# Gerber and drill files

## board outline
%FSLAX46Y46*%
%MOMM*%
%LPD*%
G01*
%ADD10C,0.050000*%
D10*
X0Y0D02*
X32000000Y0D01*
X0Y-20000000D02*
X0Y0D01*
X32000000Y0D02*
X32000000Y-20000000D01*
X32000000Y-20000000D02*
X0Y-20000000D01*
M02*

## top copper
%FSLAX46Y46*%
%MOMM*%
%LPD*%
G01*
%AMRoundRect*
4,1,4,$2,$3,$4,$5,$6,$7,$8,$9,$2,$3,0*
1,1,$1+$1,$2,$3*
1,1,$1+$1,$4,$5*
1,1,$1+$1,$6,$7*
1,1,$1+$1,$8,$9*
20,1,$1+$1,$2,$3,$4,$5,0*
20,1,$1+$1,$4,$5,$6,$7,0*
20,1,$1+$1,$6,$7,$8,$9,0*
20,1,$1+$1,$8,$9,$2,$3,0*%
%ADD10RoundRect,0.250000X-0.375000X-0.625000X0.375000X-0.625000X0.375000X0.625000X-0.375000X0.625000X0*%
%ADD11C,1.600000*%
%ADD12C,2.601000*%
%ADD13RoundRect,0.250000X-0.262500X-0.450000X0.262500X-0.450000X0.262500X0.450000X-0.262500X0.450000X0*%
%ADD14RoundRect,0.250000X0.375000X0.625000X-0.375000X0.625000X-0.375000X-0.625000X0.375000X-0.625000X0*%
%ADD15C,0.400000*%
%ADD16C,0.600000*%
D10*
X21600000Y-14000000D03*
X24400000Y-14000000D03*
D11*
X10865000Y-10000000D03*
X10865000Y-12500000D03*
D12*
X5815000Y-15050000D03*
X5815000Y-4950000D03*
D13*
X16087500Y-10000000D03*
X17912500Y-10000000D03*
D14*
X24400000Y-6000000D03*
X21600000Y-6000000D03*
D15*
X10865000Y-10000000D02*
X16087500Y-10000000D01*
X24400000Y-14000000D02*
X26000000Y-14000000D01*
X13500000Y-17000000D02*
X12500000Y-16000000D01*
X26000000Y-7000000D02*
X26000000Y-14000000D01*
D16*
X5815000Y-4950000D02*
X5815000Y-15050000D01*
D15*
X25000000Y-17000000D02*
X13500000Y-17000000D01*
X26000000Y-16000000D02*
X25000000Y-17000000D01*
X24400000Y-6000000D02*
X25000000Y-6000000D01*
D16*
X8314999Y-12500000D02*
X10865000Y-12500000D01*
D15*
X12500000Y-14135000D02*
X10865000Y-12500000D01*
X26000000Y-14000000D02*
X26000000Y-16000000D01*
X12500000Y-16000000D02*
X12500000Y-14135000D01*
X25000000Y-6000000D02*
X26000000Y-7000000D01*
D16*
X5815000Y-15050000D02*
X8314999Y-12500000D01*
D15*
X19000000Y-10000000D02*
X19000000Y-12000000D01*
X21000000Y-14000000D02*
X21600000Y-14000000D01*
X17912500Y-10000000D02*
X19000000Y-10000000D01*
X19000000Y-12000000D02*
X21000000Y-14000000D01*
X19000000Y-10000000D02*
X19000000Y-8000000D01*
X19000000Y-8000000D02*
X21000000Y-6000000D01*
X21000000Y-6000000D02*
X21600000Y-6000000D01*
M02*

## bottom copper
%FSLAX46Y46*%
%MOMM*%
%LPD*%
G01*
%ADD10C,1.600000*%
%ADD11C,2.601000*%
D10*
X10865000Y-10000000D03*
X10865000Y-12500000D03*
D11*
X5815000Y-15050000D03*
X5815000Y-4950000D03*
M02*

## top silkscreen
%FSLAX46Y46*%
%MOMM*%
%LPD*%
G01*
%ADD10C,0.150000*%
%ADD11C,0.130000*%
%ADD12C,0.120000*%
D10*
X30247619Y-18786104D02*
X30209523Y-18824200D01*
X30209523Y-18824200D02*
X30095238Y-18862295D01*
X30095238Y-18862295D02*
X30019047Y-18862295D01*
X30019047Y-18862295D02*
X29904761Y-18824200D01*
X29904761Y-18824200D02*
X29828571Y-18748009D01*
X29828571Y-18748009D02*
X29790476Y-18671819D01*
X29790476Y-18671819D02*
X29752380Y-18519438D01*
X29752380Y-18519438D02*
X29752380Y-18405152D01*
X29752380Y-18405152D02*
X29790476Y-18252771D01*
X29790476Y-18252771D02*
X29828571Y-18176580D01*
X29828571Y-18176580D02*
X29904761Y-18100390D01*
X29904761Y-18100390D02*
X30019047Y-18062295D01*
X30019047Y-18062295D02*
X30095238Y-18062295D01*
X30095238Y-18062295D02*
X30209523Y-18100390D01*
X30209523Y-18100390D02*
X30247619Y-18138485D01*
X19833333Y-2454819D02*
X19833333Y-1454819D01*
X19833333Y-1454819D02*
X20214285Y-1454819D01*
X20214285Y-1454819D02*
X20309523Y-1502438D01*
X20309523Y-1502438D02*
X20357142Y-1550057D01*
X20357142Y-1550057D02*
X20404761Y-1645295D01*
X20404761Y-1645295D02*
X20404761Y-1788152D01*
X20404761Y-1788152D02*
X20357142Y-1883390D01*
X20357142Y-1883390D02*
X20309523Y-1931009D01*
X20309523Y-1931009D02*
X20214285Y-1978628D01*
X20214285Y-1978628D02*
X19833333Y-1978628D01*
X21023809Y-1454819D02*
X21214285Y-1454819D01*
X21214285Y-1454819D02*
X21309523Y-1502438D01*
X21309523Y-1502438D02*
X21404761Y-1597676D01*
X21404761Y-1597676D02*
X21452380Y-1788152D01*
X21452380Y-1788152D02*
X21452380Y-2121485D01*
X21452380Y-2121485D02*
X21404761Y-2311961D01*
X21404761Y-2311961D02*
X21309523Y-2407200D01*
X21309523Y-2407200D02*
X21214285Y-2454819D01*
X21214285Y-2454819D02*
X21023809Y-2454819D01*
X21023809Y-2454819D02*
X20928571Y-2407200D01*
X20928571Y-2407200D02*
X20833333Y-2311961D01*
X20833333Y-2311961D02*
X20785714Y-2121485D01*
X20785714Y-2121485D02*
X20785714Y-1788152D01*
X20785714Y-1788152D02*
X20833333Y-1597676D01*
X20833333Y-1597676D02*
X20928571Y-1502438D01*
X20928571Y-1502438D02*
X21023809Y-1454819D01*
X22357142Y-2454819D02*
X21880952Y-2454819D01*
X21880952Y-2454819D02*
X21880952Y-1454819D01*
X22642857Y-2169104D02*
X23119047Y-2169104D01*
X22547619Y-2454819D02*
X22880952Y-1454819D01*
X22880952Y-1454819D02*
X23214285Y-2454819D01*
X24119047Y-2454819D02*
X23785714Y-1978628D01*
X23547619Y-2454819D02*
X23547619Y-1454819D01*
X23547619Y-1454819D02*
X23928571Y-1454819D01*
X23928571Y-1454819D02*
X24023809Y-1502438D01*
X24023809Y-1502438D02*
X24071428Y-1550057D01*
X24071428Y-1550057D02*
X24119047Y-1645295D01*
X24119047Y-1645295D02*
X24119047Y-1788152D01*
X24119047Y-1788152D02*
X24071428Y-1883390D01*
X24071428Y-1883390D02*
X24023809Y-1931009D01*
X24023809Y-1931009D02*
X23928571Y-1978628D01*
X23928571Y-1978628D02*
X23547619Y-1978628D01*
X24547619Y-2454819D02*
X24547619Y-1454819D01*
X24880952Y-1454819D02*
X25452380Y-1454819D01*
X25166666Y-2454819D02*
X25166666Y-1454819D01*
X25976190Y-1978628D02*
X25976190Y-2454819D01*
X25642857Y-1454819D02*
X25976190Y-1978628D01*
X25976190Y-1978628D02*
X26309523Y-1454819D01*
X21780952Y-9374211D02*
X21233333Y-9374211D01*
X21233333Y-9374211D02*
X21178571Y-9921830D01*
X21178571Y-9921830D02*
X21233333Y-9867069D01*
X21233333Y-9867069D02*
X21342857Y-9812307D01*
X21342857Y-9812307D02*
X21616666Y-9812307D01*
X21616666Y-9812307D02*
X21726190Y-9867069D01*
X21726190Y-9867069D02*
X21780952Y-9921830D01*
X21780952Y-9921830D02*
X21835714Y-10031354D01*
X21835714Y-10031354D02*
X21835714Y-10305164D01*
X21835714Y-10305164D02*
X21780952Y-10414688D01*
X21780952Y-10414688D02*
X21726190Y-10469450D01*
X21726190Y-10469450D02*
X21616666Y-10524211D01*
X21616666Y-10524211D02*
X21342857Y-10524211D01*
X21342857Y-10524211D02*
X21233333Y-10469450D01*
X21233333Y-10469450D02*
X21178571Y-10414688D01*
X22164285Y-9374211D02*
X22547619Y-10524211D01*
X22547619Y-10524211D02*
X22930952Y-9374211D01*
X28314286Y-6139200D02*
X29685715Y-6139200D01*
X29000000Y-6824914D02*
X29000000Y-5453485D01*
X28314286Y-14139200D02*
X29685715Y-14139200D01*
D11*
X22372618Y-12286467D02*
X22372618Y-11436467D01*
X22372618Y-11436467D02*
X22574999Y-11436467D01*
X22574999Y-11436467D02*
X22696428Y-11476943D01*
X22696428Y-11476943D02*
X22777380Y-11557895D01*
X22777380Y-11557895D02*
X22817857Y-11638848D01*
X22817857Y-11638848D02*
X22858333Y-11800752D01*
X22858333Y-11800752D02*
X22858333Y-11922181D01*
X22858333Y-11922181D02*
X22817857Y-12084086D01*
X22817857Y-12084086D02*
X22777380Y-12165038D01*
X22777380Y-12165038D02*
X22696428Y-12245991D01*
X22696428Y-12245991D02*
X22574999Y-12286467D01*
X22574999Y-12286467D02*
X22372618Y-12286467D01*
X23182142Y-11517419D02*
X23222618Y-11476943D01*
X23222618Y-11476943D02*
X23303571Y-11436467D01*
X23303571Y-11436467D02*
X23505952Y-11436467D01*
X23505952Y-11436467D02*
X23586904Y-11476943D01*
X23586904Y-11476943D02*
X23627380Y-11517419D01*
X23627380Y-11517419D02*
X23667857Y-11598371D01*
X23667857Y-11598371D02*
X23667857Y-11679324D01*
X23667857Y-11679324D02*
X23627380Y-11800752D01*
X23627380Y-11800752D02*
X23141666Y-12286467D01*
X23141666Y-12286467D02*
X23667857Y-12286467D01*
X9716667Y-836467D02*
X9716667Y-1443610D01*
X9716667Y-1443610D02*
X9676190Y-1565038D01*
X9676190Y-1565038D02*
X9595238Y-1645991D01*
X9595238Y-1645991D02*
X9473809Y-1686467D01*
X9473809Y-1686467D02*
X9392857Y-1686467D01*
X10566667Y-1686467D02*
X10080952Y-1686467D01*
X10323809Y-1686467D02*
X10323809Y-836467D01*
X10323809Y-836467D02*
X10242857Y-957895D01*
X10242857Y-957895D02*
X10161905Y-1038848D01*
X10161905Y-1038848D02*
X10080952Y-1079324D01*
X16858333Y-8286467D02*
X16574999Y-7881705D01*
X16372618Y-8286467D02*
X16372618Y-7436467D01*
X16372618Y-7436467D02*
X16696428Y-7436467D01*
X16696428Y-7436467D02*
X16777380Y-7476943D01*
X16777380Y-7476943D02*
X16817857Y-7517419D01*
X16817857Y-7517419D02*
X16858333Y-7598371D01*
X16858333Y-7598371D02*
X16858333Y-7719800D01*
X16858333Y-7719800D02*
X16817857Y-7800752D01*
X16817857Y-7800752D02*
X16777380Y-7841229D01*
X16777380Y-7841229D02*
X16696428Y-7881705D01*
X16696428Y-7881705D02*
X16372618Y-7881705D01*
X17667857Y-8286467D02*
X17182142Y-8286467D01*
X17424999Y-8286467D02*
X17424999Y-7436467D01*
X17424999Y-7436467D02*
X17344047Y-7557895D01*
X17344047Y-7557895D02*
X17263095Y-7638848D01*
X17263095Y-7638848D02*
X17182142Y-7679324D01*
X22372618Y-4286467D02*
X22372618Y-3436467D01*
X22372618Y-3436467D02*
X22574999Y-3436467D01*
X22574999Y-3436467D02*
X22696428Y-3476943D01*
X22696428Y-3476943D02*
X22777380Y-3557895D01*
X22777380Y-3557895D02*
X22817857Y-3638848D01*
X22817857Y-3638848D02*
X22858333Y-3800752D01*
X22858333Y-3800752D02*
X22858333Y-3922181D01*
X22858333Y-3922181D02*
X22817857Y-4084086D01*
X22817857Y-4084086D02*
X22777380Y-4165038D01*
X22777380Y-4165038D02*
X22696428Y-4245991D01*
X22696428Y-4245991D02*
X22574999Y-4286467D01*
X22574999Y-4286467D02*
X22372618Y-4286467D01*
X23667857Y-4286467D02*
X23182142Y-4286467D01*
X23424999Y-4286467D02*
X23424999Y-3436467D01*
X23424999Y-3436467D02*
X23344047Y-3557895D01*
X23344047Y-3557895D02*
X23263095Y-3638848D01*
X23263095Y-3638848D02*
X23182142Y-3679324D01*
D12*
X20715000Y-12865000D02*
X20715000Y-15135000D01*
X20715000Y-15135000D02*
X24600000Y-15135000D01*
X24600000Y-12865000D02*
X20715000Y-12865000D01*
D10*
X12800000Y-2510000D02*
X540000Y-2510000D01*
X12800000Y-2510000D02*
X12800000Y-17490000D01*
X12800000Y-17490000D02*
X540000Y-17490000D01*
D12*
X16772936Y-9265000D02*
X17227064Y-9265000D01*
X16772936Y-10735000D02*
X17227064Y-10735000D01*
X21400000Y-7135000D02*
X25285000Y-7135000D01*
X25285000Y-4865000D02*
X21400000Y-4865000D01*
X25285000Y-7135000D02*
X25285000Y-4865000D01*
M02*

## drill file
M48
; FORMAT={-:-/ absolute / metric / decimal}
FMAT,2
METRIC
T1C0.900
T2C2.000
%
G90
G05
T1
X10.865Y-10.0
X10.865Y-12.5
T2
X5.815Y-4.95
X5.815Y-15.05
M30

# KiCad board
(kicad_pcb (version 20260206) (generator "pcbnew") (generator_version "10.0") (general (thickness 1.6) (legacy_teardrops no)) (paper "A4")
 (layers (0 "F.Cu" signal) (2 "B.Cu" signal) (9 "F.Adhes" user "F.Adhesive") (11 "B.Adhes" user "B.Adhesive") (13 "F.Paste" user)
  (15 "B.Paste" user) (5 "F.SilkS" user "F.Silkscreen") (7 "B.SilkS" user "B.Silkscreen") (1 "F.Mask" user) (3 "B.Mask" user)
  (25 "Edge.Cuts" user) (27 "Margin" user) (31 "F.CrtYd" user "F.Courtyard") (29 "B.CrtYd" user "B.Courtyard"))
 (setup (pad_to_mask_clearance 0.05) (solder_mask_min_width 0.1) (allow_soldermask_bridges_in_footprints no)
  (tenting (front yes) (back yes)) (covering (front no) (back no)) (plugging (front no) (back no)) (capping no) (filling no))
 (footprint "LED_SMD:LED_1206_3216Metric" (layer "F.Cu") (at 23 14)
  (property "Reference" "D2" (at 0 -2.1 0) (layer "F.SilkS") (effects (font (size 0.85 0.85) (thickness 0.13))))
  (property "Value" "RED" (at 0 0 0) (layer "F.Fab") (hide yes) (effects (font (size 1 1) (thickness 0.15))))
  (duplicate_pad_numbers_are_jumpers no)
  (fp_line (start -2.285 -1.135) (end -2.285 1.135) (stroke (width 0.12) (type solid)) (layer "F.SilkS"))
  (fp_line (start -2.285 1.135) (end 1.6 1.135) (stroke (width 0.12) (type solid)) (layer "F.SilkS"))
  (fp_line (start 1.6 -1.135) (end -2.285 -1.135) (stroke (width 0.12) (type solid)) (layer "F.SilkS"))
  (pad "1" smd roundrect (at -1.4 0) (size 1.25 1.75) (layers "F.Cu" "F.Mask" "F.Paste") (roundrect_rratio 0.2) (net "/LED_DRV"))
  (pad "2" smd roundrect (at 1.4 0) (size 1.25 1.75) (layers "F.Cu" "F.Mask" "F.Paste") (roundrect_rratio 0.2) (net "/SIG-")))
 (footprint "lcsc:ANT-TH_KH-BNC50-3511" (layer "F.Cu") (at 8.34 10 -90)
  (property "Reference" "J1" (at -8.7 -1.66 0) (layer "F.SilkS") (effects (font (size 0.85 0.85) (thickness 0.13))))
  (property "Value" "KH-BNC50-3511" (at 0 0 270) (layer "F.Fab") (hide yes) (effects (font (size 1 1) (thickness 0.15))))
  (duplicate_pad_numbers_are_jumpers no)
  (fp_line (start -7.49 -4.46) (end -7.49 7.8) (stroke (width 0.15) (type default)) (layer "F.SilkS"))
  (fp_line (start -7.49 -4.46) (end 7.49 -4.46) (stroke (width 0.15) (type default)) (layer "F.SilkS"))
  (fp_line (start 7.49 -4.46) (end 7.49 7.8) (stroke (width 0.15) (type default)) (layer "F.SilkS"))
  (pad "1" thru_hole circle (at 0 -2.525 180) (size 1.6 1.6) (drill 0.9) (layers "*.Cu" "*.Mask") (remove_unused_layers no) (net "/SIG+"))
  (pad "2" thru_hole circle (at 2.5 -2.525 180) (size 1.6 1.6) (drill 0.9) (layers "*.Cu" "*.Mask") (remove_unused_layers no) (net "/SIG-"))
  (pad "3" thru_hole circle (at 5.05 2.525 90) (size 2.601 2.601) (drill 2) (layers "*.Cu" "*.Mask") (remove_unused_layers no) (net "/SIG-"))
  (pad "4" thru_hole circle (at -5.05 2.525 90) (size 2.601 2.601) (drill 2) (layers "*.Cu" "*.Mask") (remove_unused_layers no)
   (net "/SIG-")))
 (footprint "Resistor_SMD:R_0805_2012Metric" (layer "F.Cu") (at 17 10)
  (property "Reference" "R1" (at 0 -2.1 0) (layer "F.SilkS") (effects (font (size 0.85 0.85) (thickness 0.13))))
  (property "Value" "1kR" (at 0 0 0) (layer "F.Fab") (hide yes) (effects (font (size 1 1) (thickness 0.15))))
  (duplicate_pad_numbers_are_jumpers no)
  (fp_line (start -0.227064 -0.735) (end 0.227064 -0.735) (stroke (width 0.12) (type solid)) (layer "F.SilkS"))
  (fp_line (start -0.227064 0.735) (end 0.227064 0.735) (stroke (width 0.12) (type solid)) (layer "F.SilkS"))
  (pad "1" smd roundrect (at -0.9125 0) (size 1.025 1.4) (layers "F.Cu" "F.Mask" "F.Paste") (roundrect_rratio 0.243902) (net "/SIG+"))
  (pad "2" smd roundrect (at 0.9125 0) (size 1.025 1.4) (layers "F.Cu" "F.Mask" "F.Paste") (roundrect_rratio 0.243902) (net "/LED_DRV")))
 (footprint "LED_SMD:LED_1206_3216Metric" (layer "F.Cu") (at 23 6 180)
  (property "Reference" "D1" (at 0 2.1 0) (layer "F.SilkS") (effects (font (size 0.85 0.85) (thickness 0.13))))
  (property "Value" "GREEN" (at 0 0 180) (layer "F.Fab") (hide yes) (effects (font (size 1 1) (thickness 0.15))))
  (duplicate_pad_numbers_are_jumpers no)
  (fp_line (start 1.6 -1.135) (end -2.285 -1.135) (stroke (width 0.12) (type solid)) (layer "F.SilkS"))
  (fp_line (start -2.285 1.135) (end 1.6 1.135) (stroke (width 0.12) (type solid)) (layer "F.SilkS"))
  (fp_line (start -2.285 -1.135) (end -2.285 1.135) (stroke (width 0.12) (type solid)) (layer "F.SilkS"))
  (pad "1" smd roundrect (at -1.4 0 180) (size 1.25 1.75) (layers "F.Cu" "F.Mask" "F.Paste") (roundrect_rratio 0.2) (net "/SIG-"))
  (pad "2" smd roundrect (at 1.4 0 180) (size 1.25 1.75) (layers "F.Cu" "F.Mask" "F.Paste") (roundrect_rratio 0.2) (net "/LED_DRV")))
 (gr_line (start 0 0) (end 32 0) (stroke (width 0.05) (type default)) (layer "Edge.Cuts"))
 (gr_line (start 0 20) (end 0 0) (stroke (width 0.05) (type default)) (layer "Edge.Cuts"))
 (gr_line (start 32 0) (end 32 20) (stroke (width 0.05) (type default)) (layer "Edge.Cuts"))
 (gr_line (start 32 20) (end 0 20) (stroke (width 0.05) (type default)) (layer "Edge.Cuts"))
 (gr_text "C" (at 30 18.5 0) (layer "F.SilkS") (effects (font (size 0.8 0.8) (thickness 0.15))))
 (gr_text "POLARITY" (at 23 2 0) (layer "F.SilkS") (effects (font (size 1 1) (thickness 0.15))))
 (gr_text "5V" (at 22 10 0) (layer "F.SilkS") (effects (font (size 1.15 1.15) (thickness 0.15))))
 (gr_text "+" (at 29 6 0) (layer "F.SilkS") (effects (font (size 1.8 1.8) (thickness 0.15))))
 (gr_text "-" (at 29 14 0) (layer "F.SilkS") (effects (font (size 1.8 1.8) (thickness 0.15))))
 (segment (start 10.865 10) (end 16.0875 10) (width 0.4) (layer "F.Cu") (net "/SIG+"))
 (segment (start 24.4 14) (end 26 14) (width 0.4) (layer "F.Cu") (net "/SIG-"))
 (segment (start 13.5 17) (end 12.5 16) (width 0.4) (layer "F.Cu") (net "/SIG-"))
 (segment (start 26 7) (end 26 14) (width 0.4) (layer "F.Cu") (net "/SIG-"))
 (segment (start 5.815 4.95) (end 5.815 15.05) (width 0.6) (layer "F.Cu") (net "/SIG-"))
 (segment (start 25 17) (end 13.5 17) (width 0.4) (layer "F.Cu") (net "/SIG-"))
 (segment (start 26 16) (end 25 17) (width 0.4) (layer "F.Cu") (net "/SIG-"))
 (segment (start 24.4 6) (end 25 6) (width 0.4) (layer "F.Cu") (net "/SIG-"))
 (segment (start 8.314999 12.5) (end 10.865 12.5) (width 0.6) (layer "F.Cu") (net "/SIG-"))
 (segment (start 12.5 14.135) (end 10.865 12.5) (width 0.4) (layer "F.Cu") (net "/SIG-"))
 (segment (start 26 14) (end 26 16) (width 0.4) (layer "F.Cu") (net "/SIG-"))
 (segment (start 12.5 16) (end 12.5 14.135) (width 0.4) (layer "F.Cu") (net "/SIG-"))
 (segment (start 25 6) (end 26 7) (width 0.4) (layer "F.Cu") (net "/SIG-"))
 (segment (start 5.815 15.05) (end 8.314999 12.5) (width 0.6) (layer "F.Cu") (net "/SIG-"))
 (segment (start 19 10) (end 19 12) (width 0.4) (layer "F.Cu") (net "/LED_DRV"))
 (segment (start 21 14) (end 21.6 14) (width 0.4) (layer "F.Cu") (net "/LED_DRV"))
 (segment (start 17.9125 10) (end 19 10) (width 0.4) (layer "F.Cu") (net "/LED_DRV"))
 (segment (start 19 12) (end 21 14) (width 0.4) (layer "F.Cu") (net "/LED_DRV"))
 (segment (start 19 10) (end 19 8) (width 0.4) (layer "F.Cu") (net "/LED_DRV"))
 (segment (start 19 8) (end 21 6) (width 0.4) (layer "F.Cu") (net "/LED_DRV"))
 (segment (start 21 6) (end 21.6 6) (width 0.4) (layer "F.Cu") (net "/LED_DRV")))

